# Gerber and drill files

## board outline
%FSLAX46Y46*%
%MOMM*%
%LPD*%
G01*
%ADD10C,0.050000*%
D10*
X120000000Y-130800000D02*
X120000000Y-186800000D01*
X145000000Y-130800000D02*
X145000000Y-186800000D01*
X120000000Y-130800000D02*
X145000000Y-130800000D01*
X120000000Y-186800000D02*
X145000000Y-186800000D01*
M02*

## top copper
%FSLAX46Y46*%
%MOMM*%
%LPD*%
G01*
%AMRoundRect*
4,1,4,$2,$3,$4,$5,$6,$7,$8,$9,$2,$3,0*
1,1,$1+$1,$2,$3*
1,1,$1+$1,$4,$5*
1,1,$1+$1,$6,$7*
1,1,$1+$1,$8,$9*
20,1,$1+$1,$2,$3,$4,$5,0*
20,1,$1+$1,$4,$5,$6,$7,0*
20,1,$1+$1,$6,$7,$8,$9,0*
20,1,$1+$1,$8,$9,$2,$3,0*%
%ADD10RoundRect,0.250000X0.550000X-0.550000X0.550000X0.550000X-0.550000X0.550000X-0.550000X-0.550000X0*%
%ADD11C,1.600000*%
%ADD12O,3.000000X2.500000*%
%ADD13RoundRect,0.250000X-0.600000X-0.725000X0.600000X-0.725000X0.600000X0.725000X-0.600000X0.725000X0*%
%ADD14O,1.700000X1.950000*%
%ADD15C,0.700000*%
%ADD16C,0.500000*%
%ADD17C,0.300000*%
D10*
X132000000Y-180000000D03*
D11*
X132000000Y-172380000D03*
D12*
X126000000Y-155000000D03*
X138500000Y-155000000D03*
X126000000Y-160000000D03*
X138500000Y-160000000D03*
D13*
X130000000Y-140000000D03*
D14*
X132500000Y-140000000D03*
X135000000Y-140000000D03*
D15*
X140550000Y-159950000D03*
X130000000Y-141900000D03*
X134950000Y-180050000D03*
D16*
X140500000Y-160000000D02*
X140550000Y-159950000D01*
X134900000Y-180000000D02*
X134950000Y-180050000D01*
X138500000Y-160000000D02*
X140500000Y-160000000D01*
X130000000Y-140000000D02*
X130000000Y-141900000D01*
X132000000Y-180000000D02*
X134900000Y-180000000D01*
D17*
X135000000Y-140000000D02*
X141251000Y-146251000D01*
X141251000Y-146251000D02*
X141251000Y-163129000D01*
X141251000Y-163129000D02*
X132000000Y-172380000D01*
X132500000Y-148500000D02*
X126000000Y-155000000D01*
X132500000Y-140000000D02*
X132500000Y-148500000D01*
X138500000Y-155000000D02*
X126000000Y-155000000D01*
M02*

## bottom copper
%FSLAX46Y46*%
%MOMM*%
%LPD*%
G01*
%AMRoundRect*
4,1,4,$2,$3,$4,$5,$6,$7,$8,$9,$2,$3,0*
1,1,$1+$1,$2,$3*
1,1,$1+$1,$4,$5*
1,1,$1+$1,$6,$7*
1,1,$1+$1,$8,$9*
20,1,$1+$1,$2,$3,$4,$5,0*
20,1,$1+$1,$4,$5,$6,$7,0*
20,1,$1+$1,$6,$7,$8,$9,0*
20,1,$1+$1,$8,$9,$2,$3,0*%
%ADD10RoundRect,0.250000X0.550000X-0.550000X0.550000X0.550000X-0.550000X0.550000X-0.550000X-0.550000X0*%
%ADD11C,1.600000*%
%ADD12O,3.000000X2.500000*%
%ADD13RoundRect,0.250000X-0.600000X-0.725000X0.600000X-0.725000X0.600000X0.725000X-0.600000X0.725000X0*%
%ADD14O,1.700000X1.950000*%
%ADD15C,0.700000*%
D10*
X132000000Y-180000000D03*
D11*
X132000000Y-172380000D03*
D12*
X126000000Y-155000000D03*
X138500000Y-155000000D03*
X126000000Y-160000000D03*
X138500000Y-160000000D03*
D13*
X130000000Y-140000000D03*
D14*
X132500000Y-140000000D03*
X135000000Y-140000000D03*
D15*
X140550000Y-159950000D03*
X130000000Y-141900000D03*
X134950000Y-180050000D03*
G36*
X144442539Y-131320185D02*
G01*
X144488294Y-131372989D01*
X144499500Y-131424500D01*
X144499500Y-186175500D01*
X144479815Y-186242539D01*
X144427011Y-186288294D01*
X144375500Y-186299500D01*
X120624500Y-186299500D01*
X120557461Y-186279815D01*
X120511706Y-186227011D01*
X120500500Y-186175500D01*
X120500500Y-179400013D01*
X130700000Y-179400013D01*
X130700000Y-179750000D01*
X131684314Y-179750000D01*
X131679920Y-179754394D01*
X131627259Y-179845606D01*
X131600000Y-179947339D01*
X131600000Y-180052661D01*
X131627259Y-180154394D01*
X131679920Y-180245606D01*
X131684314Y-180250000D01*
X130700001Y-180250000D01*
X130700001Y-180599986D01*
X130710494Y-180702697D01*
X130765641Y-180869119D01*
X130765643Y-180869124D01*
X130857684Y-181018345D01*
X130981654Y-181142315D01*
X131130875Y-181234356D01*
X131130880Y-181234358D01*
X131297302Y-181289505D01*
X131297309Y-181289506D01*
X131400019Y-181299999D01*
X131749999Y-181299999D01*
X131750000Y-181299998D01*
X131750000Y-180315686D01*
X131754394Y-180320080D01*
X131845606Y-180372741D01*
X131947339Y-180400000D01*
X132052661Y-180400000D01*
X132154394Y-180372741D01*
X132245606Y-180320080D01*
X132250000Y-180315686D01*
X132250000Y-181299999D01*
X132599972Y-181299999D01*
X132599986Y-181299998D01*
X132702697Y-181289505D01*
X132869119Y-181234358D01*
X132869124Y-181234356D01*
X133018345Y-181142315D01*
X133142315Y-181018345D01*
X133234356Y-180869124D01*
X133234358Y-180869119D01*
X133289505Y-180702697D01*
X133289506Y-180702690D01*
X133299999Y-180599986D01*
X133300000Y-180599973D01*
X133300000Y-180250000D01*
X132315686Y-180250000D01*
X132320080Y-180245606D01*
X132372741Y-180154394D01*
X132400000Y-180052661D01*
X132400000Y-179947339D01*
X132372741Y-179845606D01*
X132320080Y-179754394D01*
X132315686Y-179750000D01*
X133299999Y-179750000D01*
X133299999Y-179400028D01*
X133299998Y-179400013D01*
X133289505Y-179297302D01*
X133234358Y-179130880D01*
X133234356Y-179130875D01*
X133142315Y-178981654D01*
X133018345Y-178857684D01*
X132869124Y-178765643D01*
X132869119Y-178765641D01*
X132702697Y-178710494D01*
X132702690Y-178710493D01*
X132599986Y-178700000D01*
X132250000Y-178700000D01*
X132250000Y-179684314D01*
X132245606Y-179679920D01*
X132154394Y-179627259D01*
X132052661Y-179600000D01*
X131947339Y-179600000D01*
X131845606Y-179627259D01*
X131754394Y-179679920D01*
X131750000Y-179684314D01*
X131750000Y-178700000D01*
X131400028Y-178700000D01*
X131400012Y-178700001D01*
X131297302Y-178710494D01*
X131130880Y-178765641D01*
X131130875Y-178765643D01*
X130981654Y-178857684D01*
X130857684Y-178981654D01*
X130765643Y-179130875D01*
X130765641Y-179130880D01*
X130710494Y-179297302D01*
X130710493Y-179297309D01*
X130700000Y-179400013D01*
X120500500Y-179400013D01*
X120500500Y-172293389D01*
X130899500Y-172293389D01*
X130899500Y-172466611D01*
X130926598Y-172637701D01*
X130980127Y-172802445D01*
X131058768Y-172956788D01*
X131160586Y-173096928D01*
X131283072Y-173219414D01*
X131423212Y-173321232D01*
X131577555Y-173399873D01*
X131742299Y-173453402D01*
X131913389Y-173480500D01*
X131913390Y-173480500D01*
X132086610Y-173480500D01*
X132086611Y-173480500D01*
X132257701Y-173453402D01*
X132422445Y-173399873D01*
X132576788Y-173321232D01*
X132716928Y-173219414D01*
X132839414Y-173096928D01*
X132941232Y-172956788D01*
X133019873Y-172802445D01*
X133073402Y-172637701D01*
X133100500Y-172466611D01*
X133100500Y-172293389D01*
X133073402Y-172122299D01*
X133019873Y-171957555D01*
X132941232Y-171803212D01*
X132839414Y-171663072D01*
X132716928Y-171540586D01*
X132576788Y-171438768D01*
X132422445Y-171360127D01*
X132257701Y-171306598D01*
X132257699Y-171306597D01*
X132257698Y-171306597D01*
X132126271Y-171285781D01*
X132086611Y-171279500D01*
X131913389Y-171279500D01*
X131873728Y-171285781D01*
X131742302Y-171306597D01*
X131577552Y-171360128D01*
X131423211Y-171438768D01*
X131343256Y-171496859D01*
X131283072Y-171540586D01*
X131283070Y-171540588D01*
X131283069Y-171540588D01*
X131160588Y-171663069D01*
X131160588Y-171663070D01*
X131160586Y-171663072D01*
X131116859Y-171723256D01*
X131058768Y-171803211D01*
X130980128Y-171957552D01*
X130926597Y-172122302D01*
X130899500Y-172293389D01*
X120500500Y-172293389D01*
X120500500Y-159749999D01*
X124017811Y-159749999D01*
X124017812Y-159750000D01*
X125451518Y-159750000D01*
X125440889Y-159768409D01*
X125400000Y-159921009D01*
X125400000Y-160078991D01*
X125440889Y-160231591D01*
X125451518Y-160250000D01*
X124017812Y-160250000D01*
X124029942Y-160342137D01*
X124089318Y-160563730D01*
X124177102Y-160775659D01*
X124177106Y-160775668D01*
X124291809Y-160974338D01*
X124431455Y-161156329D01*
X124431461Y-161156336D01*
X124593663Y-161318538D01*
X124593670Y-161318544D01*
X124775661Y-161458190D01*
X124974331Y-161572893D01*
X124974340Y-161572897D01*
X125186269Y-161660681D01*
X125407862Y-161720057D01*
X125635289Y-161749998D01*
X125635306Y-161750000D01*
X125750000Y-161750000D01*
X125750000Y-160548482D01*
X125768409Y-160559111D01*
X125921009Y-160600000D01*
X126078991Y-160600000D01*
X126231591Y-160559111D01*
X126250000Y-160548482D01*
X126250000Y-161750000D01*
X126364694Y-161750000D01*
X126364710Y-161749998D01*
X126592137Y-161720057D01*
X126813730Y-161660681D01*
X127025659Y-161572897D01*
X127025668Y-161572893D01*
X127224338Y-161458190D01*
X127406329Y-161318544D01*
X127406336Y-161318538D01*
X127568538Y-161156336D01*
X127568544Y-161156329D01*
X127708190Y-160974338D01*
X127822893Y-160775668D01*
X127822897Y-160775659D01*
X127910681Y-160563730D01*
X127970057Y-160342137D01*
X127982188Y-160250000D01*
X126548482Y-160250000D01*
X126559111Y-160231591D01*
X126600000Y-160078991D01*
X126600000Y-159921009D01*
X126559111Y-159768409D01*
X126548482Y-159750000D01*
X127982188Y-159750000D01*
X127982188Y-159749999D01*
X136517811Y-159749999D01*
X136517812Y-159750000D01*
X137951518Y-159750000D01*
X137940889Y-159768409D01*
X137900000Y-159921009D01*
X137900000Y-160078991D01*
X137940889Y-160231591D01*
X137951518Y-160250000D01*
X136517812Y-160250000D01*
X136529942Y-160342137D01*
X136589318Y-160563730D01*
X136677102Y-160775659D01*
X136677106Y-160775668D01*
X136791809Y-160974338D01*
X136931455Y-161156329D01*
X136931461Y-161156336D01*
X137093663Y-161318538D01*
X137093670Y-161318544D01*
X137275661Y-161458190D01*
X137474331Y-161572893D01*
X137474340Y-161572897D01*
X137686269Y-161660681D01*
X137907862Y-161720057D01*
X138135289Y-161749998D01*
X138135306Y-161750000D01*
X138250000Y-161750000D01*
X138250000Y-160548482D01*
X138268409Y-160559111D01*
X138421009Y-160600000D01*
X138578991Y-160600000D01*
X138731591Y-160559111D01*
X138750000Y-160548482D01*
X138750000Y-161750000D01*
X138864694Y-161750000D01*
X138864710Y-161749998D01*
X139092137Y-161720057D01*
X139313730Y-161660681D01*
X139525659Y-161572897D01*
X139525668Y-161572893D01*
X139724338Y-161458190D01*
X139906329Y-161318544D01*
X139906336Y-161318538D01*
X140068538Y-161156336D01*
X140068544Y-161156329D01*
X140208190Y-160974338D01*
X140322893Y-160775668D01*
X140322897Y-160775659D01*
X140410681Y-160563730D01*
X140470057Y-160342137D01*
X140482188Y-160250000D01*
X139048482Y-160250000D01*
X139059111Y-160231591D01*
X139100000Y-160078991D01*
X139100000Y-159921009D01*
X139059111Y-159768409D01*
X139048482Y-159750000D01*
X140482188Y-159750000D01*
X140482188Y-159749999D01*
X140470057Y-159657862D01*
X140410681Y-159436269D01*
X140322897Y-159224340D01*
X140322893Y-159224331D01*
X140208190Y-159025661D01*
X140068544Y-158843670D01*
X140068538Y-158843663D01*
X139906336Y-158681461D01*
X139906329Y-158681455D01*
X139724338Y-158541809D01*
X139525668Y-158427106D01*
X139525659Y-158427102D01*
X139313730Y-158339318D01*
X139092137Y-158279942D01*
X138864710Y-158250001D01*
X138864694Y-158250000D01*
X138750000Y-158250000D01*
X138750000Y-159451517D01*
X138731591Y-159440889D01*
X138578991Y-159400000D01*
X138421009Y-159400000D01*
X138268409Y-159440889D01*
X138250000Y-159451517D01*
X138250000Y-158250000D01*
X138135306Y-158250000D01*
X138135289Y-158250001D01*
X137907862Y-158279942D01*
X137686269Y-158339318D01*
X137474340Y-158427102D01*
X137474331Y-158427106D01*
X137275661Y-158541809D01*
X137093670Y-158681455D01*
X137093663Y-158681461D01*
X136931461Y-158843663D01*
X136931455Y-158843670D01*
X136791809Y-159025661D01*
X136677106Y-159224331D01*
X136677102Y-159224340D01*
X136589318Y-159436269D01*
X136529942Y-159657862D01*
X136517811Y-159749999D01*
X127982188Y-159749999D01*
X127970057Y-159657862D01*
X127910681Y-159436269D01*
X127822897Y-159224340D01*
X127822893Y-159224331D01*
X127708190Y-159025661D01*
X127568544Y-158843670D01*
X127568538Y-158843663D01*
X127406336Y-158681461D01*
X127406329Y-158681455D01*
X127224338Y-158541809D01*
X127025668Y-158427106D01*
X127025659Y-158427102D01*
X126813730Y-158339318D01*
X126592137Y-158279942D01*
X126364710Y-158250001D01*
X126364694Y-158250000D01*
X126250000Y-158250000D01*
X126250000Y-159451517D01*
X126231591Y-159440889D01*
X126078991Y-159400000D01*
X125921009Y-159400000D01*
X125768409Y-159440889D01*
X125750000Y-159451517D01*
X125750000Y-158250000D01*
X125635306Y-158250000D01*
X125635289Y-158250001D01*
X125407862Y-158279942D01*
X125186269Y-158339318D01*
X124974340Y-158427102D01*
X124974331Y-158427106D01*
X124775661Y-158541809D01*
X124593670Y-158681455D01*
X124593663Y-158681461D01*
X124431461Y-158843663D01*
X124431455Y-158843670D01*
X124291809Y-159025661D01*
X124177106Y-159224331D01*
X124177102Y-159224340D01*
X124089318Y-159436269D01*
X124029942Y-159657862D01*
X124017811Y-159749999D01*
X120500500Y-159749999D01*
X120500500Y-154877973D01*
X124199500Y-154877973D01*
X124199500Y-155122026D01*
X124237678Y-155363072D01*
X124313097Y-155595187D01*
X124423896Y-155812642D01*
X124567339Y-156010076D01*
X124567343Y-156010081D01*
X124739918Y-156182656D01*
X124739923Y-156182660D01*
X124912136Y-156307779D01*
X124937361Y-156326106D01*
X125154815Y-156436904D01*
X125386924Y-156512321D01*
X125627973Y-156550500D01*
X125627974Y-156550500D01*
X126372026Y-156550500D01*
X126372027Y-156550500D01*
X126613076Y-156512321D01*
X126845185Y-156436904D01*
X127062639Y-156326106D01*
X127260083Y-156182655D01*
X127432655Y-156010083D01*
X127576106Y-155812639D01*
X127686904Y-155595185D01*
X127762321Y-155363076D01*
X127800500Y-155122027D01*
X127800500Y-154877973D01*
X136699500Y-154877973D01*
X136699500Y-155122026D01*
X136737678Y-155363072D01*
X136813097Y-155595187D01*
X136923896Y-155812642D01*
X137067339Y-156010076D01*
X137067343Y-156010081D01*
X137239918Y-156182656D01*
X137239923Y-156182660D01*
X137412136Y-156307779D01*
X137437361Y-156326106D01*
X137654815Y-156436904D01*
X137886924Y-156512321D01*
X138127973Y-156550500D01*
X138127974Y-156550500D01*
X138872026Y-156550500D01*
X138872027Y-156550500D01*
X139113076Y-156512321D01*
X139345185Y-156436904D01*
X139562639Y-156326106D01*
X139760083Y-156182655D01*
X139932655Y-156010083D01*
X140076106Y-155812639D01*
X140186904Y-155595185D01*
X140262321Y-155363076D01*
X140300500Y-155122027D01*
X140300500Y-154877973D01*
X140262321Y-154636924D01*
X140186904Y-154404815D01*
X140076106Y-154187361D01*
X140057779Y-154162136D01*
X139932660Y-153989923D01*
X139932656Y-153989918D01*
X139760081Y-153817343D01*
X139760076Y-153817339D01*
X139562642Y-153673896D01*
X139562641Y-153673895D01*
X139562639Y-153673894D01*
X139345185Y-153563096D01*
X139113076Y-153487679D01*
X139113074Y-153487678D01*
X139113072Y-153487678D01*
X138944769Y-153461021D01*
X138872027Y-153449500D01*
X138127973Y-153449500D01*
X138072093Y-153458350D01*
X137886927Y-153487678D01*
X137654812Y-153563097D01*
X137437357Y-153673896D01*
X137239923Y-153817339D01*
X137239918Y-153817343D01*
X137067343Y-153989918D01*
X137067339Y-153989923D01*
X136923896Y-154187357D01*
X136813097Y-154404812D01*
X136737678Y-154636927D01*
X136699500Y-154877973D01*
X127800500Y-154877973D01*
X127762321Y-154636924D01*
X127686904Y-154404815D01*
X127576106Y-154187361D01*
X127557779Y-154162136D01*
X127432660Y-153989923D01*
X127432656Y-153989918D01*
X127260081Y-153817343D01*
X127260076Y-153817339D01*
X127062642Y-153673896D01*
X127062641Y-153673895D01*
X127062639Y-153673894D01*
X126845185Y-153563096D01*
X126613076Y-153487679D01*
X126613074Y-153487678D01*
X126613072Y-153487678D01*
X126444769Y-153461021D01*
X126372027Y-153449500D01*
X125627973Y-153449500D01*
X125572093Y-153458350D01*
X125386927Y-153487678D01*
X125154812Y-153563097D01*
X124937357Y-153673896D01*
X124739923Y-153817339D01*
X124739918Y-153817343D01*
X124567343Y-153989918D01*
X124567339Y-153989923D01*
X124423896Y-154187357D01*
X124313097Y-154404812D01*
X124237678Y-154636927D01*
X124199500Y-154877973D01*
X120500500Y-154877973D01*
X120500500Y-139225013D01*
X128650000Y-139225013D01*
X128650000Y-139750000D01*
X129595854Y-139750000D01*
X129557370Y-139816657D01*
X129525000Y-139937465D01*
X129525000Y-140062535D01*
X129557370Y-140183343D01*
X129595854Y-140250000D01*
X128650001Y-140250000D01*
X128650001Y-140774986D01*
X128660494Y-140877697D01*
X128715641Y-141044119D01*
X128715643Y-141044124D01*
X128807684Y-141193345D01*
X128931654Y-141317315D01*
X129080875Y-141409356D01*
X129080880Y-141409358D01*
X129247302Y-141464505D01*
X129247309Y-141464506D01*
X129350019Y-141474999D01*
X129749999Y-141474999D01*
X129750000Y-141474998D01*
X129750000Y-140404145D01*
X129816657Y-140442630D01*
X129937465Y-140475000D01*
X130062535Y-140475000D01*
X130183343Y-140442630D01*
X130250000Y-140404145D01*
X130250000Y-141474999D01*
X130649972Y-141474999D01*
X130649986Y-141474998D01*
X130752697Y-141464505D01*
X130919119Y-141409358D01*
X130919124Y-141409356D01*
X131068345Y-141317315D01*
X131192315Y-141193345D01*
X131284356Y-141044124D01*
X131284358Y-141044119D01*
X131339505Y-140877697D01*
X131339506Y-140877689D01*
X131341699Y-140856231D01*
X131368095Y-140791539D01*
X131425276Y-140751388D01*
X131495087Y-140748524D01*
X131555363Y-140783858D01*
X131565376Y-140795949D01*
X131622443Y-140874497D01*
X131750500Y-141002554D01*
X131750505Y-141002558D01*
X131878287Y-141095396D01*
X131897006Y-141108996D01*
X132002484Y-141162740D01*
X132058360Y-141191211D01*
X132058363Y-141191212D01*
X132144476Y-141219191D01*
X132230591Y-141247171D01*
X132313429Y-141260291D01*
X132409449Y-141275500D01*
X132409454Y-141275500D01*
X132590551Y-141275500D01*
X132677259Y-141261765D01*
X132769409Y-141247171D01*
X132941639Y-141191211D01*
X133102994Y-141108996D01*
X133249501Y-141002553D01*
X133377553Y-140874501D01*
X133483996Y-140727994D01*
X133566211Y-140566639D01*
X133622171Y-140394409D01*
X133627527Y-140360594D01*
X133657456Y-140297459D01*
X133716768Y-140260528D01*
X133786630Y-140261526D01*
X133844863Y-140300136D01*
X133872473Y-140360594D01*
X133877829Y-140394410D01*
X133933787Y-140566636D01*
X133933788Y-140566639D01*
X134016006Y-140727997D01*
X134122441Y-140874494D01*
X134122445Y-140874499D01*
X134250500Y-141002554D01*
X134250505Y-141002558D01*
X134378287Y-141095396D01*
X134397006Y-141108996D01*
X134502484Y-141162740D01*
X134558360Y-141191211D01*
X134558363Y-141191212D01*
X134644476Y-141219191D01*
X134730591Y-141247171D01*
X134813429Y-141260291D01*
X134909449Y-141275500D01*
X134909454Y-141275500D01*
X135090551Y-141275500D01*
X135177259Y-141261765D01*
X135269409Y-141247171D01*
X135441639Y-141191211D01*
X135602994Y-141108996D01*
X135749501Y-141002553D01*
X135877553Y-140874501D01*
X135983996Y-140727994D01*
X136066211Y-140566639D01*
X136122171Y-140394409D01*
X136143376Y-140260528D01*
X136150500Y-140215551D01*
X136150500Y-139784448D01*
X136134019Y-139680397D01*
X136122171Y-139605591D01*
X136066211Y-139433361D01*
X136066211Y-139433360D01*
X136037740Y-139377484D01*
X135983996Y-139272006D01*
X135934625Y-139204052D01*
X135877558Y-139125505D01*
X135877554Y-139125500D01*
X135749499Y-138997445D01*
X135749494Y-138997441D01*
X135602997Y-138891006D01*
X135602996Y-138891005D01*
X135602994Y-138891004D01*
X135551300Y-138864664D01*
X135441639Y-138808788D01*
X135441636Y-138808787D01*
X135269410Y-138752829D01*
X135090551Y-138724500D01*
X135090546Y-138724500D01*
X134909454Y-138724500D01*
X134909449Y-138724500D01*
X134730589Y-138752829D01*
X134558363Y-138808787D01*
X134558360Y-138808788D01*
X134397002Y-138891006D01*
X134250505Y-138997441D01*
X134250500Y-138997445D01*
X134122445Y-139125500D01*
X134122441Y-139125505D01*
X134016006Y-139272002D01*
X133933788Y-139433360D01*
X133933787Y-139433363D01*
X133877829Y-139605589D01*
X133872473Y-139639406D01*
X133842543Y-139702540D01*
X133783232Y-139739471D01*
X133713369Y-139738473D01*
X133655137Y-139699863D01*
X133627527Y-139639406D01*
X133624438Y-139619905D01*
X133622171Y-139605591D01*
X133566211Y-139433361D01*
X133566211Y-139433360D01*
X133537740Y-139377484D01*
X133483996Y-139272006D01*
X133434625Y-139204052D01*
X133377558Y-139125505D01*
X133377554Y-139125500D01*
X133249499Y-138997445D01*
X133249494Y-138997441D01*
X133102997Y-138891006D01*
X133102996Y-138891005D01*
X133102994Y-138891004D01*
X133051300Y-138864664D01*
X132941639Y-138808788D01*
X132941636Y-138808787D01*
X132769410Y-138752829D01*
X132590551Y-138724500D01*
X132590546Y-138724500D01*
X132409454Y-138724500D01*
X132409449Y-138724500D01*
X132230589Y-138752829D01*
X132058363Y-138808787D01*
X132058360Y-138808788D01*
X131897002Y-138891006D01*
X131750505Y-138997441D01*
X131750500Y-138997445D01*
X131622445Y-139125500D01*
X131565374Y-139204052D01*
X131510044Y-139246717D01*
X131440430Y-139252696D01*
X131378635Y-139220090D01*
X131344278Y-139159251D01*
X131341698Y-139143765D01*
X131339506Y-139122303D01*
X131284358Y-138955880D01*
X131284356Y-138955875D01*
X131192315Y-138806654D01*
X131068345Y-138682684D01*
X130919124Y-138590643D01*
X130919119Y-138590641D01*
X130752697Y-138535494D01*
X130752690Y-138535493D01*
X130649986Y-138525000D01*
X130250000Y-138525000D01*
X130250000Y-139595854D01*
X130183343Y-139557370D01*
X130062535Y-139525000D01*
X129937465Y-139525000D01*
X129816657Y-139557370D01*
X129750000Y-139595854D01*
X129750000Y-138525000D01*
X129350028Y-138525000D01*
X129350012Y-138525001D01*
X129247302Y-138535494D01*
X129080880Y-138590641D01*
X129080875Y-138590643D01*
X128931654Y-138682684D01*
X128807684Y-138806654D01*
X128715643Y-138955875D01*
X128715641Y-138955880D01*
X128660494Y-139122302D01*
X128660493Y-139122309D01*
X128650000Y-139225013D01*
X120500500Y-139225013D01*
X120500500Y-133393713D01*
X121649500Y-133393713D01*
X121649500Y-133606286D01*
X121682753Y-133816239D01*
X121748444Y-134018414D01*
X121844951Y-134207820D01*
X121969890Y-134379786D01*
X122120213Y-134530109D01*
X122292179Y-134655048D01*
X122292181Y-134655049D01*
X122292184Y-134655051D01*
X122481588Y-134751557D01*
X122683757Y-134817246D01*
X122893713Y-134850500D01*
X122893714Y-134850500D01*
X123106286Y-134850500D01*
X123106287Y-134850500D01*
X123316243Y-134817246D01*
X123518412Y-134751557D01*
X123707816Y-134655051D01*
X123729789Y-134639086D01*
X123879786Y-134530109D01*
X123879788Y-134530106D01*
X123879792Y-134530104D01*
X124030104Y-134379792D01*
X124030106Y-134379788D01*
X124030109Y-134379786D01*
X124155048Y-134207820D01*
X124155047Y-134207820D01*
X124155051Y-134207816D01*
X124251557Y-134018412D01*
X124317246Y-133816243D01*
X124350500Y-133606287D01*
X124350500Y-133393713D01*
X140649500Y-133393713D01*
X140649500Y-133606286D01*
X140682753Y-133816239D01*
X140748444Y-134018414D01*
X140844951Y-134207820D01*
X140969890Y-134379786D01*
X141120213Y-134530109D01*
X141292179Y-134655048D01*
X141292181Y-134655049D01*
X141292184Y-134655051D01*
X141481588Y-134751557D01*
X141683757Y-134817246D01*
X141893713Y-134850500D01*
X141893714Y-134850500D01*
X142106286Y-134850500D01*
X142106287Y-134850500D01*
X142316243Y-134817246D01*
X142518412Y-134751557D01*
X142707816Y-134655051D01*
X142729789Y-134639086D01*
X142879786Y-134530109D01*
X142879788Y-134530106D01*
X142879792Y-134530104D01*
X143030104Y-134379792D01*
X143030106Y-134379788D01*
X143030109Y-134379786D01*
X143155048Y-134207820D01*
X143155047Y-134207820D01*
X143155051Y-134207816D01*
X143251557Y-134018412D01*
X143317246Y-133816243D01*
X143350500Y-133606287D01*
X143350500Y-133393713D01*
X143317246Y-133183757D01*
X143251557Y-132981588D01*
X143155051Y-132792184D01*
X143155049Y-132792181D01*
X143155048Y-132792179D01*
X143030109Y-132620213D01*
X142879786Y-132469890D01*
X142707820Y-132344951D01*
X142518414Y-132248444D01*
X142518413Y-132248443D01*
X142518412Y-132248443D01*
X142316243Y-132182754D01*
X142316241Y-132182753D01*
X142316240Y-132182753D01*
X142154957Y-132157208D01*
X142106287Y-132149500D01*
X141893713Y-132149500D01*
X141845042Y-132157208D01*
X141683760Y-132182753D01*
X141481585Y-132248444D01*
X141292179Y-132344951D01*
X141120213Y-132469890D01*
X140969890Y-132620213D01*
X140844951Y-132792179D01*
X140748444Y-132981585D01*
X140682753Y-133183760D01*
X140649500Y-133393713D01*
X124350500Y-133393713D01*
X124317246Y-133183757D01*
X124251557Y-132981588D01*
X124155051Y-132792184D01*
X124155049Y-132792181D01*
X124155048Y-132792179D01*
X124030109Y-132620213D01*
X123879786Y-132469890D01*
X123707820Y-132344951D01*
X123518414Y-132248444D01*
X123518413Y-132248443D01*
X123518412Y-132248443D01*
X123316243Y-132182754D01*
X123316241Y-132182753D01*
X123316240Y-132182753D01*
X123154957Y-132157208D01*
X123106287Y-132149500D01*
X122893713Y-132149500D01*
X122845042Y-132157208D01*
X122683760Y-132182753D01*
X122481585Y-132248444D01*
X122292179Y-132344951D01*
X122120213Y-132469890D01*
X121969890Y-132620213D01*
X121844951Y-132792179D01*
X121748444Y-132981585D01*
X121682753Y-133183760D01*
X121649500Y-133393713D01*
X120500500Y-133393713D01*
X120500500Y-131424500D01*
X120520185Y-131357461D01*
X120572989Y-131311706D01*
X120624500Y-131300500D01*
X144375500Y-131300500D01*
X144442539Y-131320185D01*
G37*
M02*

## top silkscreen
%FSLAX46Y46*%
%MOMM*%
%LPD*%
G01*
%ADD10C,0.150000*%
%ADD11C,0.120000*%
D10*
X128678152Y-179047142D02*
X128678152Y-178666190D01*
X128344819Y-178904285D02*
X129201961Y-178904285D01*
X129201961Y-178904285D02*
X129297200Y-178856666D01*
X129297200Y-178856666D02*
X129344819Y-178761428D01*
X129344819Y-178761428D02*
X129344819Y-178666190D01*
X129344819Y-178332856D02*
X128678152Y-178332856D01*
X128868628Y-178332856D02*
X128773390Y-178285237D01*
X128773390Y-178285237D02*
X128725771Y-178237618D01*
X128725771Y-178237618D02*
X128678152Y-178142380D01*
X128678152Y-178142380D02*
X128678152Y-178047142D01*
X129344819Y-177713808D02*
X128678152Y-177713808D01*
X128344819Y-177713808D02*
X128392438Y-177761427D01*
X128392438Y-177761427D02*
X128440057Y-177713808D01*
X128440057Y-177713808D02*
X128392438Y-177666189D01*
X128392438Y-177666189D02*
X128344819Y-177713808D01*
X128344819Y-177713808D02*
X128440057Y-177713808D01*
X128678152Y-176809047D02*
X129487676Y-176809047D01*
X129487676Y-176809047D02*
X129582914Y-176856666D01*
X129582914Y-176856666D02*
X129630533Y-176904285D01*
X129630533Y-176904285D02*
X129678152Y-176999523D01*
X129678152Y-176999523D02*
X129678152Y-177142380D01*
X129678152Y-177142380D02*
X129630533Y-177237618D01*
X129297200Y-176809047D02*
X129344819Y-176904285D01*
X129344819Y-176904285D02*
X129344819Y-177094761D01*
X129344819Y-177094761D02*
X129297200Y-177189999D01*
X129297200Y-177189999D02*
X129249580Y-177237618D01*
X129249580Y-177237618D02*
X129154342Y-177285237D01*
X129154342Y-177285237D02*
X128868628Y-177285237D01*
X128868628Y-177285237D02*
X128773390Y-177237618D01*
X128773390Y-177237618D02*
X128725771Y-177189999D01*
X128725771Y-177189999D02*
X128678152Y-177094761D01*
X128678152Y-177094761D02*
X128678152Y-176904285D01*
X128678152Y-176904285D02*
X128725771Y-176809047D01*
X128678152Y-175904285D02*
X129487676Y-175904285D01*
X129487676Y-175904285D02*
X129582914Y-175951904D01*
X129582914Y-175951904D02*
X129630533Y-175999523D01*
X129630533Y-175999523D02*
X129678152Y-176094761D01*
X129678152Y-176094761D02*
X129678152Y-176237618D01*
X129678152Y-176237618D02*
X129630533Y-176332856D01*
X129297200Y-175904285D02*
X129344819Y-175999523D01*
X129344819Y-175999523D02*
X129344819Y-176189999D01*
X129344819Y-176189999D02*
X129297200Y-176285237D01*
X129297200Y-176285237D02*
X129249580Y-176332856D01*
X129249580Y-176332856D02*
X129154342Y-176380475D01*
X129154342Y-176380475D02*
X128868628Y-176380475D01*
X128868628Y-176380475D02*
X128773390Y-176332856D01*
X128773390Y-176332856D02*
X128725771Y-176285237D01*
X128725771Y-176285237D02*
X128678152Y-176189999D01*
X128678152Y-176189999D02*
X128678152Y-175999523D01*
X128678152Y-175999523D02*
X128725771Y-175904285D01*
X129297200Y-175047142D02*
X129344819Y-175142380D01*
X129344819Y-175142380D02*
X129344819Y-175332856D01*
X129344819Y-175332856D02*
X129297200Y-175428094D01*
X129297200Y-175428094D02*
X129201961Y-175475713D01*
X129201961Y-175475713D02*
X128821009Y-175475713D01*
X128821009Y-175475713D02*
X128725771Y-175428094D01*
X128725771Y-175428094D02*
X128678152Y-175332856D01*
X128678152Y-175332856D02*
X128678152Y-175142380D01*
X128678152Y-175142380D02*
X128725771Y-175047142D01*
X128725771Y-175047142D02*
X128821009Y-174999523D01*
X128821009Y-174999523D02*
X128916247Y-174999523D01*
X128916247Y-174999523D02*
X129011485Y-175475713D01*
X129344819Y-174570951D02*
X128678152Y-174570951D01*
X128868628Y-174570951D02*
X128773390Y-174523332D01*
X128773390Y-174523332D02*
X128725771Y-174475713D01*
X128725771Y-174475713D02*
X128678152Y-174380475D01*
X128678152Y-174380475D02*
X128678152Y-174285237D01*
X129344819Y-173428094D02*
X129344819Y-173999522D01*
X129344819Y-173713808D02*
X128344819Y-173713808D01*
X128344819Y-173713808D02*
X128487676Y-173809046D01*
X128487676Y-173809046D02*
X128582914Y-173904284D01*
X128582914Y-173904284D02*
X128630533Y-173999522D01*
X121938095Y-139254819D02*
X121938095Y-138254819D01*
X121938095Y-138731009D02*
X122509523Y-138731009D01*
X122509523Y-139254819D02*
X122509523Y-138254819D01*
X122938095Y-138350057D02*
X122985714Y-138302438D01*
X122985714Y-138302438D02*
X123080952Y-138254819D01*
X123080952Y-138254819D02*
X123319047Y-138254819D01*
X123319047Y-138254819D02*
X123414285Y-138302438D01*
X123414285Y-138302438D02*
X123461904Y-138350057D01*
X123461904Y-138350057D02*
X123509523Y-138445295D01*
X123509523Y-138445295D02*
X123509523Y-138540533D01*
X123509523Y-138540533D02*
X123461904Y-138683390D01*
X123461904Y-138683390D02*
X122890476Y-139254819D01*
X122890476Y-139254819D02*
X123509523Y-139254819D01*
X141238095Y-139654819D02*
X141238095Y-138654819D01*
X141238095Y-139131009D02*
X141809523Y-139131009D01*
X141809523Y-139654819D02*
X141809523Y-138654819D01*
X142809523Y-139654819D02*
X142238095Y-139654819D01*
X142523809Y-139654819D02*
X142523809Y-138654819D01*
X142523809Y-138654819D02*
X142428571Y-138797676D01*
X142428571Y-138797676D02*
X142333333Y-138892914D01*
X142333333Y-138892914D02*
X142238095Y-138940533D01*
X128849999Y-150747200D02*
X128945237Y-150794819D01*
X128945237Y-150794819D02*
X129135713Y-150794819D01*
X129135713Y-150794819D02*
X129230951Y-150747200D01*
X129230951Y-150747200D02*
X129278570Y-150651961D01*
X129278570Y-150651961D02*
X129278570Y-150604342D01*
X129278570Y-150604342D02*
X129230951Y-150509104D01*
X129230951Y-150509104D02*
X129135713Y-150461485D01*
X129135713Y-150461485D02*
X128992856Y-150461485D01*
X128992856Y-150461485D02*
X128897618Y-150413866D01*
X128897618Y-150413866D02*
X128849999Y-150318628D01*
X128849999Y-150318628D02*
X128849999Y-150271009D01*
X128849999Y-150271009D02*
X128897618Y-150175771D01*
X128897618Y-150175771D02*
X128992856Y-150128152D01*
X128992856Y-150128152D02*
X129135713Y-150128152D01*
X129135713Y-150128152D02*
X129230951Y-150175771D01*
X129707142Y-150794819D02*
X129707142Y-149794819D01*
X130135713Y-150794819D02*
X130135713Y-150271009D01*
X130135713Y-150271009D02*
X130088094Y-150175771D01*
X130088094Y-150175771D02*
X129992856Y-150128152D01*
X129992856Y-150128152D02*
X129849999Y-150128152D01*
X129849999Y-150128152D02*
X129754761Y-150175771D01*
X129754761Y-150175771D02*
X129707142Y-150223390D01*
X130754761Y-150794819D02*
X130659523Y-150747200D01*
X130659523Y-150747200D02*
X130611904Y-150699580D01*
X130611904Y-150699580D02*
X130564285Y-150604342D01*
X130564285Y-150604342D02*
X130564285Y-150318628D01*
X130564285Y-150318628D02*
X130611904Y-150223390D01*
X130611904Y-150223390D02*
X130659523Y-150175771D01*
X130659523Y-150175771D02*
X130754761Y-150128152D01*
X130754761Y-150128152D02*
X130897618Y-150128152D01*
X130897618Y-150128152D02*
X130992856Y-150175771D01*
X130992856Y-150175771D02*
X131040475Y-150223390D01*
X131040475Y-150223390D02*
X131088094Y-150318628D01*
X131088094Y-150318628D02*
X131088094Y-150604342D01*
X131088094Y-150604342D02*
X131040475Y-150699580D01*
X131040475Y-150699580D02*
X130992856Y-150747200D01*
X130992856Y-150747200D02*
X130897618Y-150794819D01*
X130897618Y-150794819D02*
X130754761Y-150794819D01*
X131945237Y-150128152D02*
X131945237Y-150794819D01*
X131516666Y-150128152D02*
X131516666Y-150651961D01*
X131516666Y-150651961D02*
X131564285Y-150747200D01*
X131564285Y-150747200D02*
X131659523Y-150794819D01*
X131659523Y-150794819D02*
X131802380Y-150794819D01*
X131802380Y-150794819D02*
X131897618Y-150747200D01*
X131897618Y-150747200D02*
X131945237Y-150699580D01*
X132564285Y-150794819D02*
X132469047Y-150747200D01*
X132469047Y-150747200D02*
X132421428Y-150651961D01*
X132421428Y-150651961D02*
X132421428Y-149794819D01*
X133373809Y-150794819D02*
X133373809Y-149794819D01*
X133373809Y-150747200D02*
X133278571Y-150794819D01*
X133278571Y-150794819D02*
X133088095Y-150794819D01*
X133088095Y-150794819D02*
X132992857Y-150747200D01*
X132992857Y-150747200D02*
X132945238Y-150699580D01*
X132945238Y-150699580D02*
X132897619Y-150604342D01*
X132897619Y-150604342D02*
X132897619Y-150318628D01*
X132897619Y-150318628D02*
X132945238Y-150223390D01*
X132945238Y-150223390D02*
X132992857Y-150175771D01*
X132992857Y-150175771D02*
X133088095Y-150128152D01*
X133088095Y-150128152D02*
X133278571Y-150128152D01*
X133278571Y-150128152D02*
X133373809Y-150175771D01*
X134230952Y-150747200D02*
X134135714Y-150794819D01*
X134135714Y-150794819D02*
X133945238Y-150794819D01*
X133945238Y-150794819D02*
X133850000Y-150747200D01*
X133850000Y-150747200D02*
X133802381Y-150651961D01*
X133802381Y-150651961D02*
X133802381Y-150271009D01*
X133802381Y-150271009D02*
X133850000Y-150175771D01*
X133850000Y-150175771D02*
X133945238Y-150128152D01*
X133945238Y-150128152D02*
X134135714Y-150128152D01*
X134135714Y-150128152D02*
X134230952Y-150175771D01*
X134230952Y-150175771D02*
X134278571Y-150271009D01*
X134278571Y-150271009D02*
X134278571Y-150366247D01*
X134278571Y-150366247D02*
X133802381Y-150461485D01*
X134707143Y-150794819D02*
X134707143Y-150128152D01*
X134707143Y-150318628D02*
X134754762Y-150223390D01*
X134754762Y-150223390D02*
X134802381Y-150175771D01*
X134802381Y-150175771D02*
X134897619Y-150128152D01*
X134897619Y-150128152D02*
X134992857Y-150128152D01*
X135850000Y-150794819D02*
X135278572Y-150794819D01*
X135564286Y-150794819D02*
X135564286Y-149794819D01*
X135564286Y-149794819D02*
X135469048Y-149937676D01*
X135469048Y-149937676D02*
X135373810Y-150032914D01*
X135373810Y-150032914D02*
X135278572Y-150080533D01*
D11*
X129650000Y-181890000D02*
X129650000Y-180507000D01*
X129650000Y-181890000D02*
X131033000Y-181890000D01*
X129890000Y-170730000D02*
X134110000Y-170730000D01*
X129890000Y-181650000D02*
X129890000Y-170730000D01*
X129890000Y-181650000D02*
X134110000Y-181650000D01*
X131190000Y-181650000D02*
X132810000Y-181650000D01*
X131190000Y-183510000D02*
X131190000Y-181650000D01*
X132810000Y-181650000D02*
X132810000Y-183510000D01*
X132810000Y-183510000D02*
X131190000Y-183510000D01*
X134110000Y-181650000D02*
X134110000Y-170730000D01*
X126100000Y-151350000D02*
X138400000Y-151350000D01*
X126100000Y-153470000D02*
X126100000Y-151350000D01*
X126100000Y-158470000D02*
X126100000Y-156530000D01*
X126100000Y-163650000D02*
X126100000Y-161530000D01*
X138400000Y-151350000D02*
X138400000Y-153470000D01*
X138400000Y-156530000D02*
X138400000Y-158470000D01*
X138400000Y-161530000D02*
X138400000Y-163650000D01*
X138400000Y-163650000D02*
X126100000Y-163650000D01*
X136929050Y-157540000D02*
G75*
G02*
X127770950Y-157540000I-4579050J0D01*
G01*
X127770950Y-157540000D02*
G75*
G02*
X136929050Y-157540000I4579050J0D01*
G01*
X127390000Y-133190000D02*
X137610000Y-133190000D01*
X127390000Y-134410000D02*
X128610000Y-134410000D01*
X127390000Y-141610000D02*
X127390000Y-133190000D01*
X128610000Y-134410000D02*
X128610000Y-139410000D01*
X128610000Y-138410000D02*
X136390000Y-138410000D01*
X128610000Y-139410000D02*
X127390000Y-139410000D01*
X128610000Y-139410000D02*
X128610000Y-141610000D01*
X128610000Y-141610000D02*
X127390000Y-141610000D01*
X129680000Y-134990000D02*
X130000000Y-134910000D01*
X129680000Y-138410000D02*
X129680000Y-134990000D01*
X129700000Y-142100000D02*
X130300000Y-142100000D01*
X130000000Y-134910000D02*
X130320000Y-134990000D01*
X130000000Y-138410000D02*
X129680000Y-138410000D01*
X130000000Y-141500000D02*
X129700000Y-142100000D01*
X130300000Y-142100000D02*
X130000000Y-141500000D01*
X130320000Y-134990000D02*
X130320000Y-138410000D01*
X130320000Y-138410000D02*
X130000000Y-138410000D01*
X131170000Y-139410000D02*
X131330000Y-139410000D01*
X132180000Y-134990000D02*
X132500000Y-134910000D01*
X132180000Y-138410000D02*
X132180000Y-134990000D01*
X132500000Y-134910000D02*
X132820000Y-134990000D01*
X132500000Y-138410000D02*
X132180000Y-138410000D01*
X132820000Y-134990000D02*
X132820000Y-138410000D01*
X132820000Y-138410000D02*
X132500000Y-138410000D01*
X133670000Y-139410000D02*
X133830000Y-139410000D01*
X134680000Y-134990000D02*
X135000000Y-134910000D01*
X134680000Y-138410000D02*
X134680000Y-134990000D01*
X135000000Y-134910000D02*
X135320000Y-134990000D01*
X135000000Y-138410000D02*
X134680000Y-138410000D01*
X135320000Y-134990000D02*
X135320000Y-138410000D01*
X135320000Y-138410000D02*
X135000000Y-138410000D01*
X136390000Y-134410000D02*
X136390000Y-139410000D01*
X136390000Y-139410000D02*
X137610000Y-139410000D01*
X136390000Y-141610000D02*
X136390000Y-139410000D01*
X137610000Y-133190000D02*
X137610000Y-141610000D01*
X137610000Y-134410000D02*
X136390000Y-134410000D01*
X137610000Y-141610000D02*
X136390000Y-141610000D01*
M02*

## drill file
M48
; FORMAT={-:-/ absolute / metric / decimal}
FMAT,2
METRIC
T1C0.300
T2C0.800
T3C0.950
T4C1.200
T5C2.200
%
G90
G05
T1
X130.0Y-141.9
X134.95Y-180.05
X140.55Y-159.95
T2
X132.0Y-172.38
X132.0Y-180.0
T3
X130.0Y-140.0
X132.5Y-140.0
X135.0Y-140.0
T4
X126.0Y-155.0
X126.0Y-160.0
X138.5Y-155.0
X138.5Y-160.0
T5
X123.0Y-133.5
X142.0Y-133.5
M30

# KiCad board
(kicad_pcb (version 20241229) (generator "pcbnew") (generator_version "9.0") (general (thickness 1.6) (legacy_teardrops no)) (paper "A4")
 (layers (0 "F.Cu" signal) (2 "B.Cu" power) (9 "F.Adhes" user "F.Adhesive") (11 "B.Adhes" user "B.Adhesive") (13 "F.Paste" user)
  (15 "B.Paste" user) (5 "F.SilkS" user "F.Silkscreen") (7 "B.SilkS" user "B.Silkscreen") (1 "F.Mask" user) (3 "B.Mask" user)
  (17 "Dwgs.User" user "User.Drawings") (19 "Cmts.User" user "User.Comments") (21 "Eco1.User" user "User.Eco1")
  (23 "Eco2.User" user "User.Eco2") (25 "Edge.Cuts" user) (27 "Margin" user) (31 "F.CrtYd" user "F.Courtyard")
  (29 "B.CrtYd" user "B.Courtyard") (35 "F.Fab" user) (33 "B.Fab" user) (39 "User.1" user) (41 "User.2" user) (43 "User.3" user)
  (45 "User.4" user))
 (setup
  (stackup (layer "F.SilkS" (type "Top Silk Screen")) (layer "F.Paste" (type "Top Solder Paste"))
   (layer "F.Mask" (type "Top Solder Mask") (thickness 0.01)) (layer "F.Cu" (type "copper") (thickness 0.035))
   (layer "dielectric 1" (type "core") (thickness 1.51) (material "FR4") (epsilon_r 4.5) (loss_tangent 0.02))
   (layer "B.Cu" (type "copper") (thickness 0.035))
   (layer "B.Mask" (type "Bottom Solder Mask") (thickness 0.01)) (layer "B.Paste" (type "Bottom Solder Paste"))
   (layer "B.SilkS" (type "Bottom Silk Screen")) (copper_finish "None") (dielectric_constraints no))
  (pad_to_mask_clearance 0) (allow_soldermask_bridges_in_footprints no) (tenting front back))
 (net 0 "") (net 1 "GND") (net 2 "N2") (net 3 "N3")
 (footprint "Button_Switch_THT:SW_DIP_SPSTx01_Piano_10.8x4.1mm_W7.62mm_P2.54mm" (layer "F.Cu") (at 132 180 90)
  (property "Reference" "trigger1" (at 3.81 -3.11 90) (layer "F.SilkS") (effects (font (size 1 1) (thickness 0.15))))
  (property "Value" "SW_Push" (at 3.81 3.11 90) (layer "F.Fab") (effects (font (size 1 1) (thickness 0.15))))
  (fp_line (start -1.89 -2.35) (end -0.507 -2.35) (stroke (width 0.12) (type solid)) (layer "F.SilkS"))
  (fp_line (start -1.89 -2.35) (end -1.89 -0.967) (stroke (width 0.12) (type solid)) (layer "F.SilkS"))
  (fp_line (start 9.27 -2.11) (end 9.27 2.11) (stroke (width 0.12) (type solid)) (layer "F.SilkS"))
  (fp_line (start -1.65 -2.11) (end 9.27 -2.11) (stroke (width 0.12) (type solid)) (layer "F.SilkS"))
  (fp_line (start -1.65 -2.11) (end -1.65 2.11) (stroke (width 0.12) (type solid)) (layer "F.SilkS"))
  (fp_line (start -1.65 -0.81) (end -1.65 0.81) (stroke (width 0.12) (type solid)) (layer "F.SilkS"))
  (fp_line (start -3.51 -0.81) (end -1.65 -0.81) (stroke (width 0.12) (type solid)) (layer "F.SilkS"))
  (fp_line (start -1.65 0.81) (end -3.51 0.81) (stroke (width 0.12) (type solid)) (layer "F.SilkS"))
  (fp_line (start -3.51 0.81) (end -3.51 -0.81) (stroke (width 0.12) (type solid)) (layer "F.SilkS"))
  (fp_line (start -1.65 2.11) (end 9.27 2.11) (stroke (width 0.12) (type solid)) (layer "F.SilkS"))
  (pad "1" thru_hole roundrect (at 0 0 90) (size 1.6 1.6) (drill 0.8) (layers "*.Cu" "*.Mask") (remove_unused_layers no)
   (roundrect_rratio 0.15625) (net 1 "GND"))
  (pad "2" thru_hole circle (at 7.62 0 90) (size 1.6 1.6) (drill 0.8) (layers "*.Cu" "*.Mask") (remove_unused_layers no) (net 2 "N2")))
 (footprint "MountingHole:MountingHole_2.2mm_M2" (layer "F.Cu") (at 123 133.5)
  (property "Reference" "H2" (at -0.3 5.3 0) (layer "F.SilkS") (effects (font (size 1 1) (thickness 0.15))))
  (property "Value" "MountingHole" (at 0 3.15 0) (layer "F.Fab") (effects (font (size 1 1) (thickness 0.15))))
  (pad "" np_thru_hole circle (at 0 0) (size 2.2 2.2) (drill 2.2) (layers "*.Cu" "*.Mask")))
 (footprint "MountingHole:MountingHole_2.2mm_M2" (layer "F.Cu") (at 142 133.5)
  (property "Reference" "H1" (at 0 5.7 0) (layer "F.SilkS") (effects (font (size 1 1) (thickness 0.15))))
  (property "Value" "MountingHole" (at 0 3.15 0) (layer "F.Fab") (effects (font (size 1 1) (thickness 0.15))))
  (pad "" np_thru_hole circle (at 0 0) (size 2.2 2.2) (drill 2.2) (layers "*.Cu" "*.Mask")))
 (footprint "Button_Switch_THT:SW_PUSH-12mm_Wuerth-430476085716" (layer "F.Cu") (at 126 155)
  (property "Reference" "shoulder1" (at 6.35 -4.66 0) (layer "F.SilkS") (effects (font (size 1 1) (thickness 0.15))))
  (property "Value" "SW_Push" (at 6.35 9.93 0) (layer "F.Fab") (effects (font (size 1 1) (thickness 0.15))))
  (fp_line (start 0.1 -3.65) (end 12.4 -3.65) (stroke (width 0.12) (type solid)) (layer "F.SilkS"))
  (fp_line (start 0.1 -1.53) (end 0.1 -3.65) (stroke (width 0.12) (type solid)) (layer "F.SilkS"))
  (fp_line (start 0.1 3.47) (end 0.1 1.53) (stroke (width 0.12) (type solid)) (layer "F.SilkS"))
  (fp_line (start 0.1 8.65) (end 0.1 6.53) (stroke (width 0.12) (type solid)) (layer "F.SilkS"))
  (fp_line (start 12.4 -3.65) (end 12.4 -1.53) (stroke (width 0.12) (type solid)) (layer "F.SilkS"))
  (fp_line (start 12.4 1.53) (end 12.4 3.47) (stroke (width 0.12) (type solid)) (layer "F.SilkS"))
  (fp_line (start 12.4 6.53) (end 12.4 8.65) (stroke (width 0.12) (type solid)) (layer "F.SilkS"))
  (fp_line (start 12.4 8.65) (end 0.1 8.65) (stroke (width 0.12) (type solid)) (layer "F.SilkS"))
  (fp_circle (center 6.35 2.54) (end 10.92905 2.54) (stroke (width 0.12) (type solid)) (fill no) (layer "F.SilkS"))
  (pad "1" thru_hole oval (at 0 0) (size 3 2.5) (drill 1.2) (layers "*.Cu" "*.Mask") (remove_unused_layers no) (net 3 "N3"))
  (pad "1" thru_hole oval (at 12.5 0) (size 3 2.5) (drill 1.2) (layers "*.Cu" "*.Mask") (remove_unused_layers no) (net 3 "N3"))
  (pad "2" thru_hole oval (at 0 5) (size 3 2.5) (drill 1.2) (layers "*.Cu" "*.Mask") (remove_unused_layers no) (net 1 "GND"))
  (pad "2" thru_hole oval (at 12.5 5) (size 3 2.5) (drill 1.2) (layers "*.Cu" "*.Mask") (remove_unused_layers no) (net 1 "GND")))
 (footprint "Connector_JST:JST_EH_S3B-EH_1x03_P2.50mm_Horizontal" (layer "F.Cu") (at 130 140)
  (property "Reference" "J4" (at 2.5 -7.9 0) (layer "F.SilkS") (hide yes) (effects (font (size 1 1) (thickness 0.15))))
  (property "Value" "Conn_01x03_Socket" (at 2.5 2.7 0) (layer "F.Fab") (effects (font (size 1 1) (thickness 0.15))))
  (fp_line (start -2.61 -6.81) (end 7.61 -6.81) (stroke (width 0.12) (type solid)) (layer "F.SilkS"))
  (fp_line (start -2.61 -5.59) (end -1.39 -5.59) (stroke (width 0.12) (type solid)) (layer "F.SilkS"))
  (fp_line (start -2.61 1.61) (end -2.61 -6.81) (stroke (width 0.12) (type solid)) (layer "F.SilkS"))
  (fp_line (start -1.39 -5.59) (end -1.39 -0.59) (stroke (width 0.12) (type solid)) (layer "F.SilkS"))
  (fp_line (start -1.39 -1.59) (end 6.39 -1.59) (stroke (width 0.12) (type solid)) (layer "F.SilkS"))
  (fp_line (start -1.39 -0.59) (end -2.61 -0.59) (stroke (width 0.12) (type solid)) (layer "F.SilkS"))
  (fp_line (start -1.39 -0.59) (end -1.39 1.61) (stroke (width 0.12) (type solid)) (layer "F.SilkS"))
  (fp_line (start -1.39 1.61) (end -2.61 1.61) (stroke (width 0.12) (type solid)) (layer "F.SilkS"))
  (fp_line (start -0.32 -5.01) (end 0 -5.09) (stroke (width 0.12) (type solid)) (layer "F.SilkS"))
  (fp_line (start -0.32 -1.59) (end -0.32 -5.01) (stroke (width 0.12) (type solid)) (layer "F.SilkS"))
  (fp_line (start -0.3 2.1) (end 0.3 2.1) (stroke (width 0.12) (type solid)) (layer "F.SilkS"))
  (fp_line (start 0 -5.09) (end 0.32 -5.01) (stroke (width 0.12) (type solid)) (layer "F.SilkS"))
  (fp_line (start 0 -1.59) (end -0.32 -1.59) (stroke (width 0.12) (type solid)) (layer "F.SilkS"))
  (fp_line (start 0 1.5) (end -0.3 2.1) (stroke (width 0.12) (type solid)) (layer "F.SilkS"))
  (fp_line (start 0.3 2.1) (end 0 1.5) (stroke (width 0.12) (type solid)) (layer "F.SilkS"))
  (fp_line (start 0.32 -5.01) (end 0.32 -1.59) (stroke (width 0.12) (type solid)) (layer "F.SilkS"))
  (fp_line (start 0.32 -1.59) (end 0 -1.59) (stroke (width 0.12) (type solid)) (layer "F.SilkS"))
  (fp_line (start 1.17 -0.59) (end 1.33 -0.59) (stroke (width 0.12) (type solid)) (layer "F.SilkS"))
  (fp_line (start 2.18 -5.01) (end 2.5 -5.09) (stroke (width 0.12) (type solid)) (layer "F.SilkS"))
  (fp_line (start 2.18 -1.59) (end 2.18 -5.01) (stroke (width 0.12) (type solid)) (layer "F.SilkS"))
  (fp_line (start 2.5 -5.09) (end 2.82 -5.01) (stroke (width 0.12) (type solid)) (layer "F.SilkS"))
  (fp_line (start 2.5 -1.59) (end 2.18 -1.59) (stroke (width 0.12) (type solid)) (layer "F.SilkS"))
  (fp_line (start 2.82 -5.01) (end 2.82 -1.59) (stroke (width 0.12) (type solid)) (layer "F.SilkS"))
  (fp_line (start 2.82 -1.59) (end 2.5 -1.59) (stroke (width 0.12) (type solid)) (layer "F.SilkS"))
  (fp_line (start 3.67 -0.59) (end 3.83 -0.59) (stroke (width 0.12) (type solid)) (layer "F.SilkS"))
  (fp_line (start 4.68 -5.01) (end 5 -5.09) (stroke (width 0.12) (type solid)) (layer "F.SilkS"))
  (fp_line (start 4.68 -1.59) (end 4.68 -5.01) (stroke (width 0.12) (type solid)) (layer "F.SilkS"))
  (fp_line (start 5 -5.09) (end 5.32 -5.01) (stroke (width 0.12) (type solid)) (layer "F.SilkS"))
  (fp_line (start 5 -1.59) (end 4.68 -1.59) (stroke (width 0.12) (type solid)) (layer "F.SilkS"))
  (fp_line (start 5.32 -5.01) (end 5.32 -1.59) (stroke (width 0.12) (type solid)) (layer "F.SilkS"))
  (fp_line (start 5.32 -1.59) (end 5 -1.59) (stroke (width 0.12) (type solid)) (layer "F.SilkS"))
  (fp_line (start 6.39 -5.59) (end 6.39 -0.59) (stroke (width 0.12) (type solid)) (layer "F.SilkS"))
  (fp_line (start 6.39 -0.59) (end 7.61 -0.59) (stroke (width 0.12) (type solid)) (layer "F.SilkS"))
  (fp_line (start 6.39 1.61) (end 6.39 -0.59) (stroke (width 0.12) (type solid)) (layer "F.SilkS"))
  (fp_line (start 7.61 -6.81) (end 7.61 1.61) (stroke (width 0.12) (type solid)) (layer "F.SilkS"))
  (fp_line (start 7.61 -5.59) (end 6.39 -5.59) (stroke (width 0.12) (type solid)) (layer "F.SilkS"))
  (fp_line (start 7.61 1.61) (end 6.39 1.61) (stroke (width 0.12) (type solid)) (layer "F.SilkS"))
  (pad "1" thru_hole roundrect (at 0 0) (size 1.7 1.95) (drill 0.95) (layers "*.Cu" "*.Mask") (remove_unused_layers no)
   (roundrect_rratio 0.147059) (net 1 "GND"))
  (pad "2" thru_hole oval (at 2.5 0) (size 1.7 1.95) (drill 0.95) (layers "*.Cu" "*.Mask") (remove_unused_layers no) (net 3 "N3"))
  (pad "3" thru_hole oval (at 5 0) (size 1.7 1.95) (drill 0.95) (layers "*.Cu" "*.Mask") (remove_unused_layers no) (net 2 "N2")))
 (gr_line (start 120 130.8) (end 120 186.8) (stroke (width 0.05) (type solid)) (layer "Edge.Cuts"))
 (gr_line (start 145 130.8) (end 145 186.8) (stroke (width 0.05) (type default)) (layer "Edge.Cuts"))
 (gr_line (start 120 130.8) (end 145 130.8) (stroke (width 0.05) (type solid)) (layer "Edge.Cuts"))
 (gr_line (start 120 186.8) (end 145 186.8) (stroke (width 0.05) (type solid)) (layer "Edge.Cuts"))
 (segment (start 140.5 160) (end 140.55 159.95) (width 0.5) (layer "F.Cu") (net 1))
 (segment (start 134.9 180) (end 134.95 180.05) (width 0.5) (layer "F.Cu") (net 1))
 (segment (start 138.5 160) (end 140.5 160) (width 0.5) (layer "F.Cu") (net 1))
 (segment (start 130 140) (end 130 141.9) (width 0.5) (layer "F.Cu") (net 1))
 (segment (start 132 180) (end 134.9 180) (width 0.5) (layer "F.Cu") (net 1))
 (via (at 140.55 159.95) (size 0.7) (drill 0.3) (layers "F.Cu" "B.Cu") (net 1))
 (via (at 130 141.9) (size 0.7) (drill 0.3) (layers "F.Cu" "B.Cu") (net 1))
 (via (at 134.95 180.05) (size 0.7) (drill 0.3) (layers "F.Cu" "B.Cu") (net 1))
 (segment (start 135 140) (end 141.251 146.251) (width 0.3) (layer "F.Cu") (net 2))
 (segment (start 141.251 146.251) (end 141.251 163.129) (width 0.3) (layer "F.Cu") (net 2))
 (segment (start 141.251 163.129) (end 132 172.38) (width 0.3) (layer "F.Cu") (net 2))
 (segment (start 132.5 148.5) (end 126 155) (width 0.3) (layer "F.Cu") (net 3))
 (segment (start 132.5 140) (end 132.5 148.5) (width 0.3) (layer "F.Cu") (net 3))
 (segment (start 138.5 155) (end 126 155) (width 0.3) (layer "F.Cu") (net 3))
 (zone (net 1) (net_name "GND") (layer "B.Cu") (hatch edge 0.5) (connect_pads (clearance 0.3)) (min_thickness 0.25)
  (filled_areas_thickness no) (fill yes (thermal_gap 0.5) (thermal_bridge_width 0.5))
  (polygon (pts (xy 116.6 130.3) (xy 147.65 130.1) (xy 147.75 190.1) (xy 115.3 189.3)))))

